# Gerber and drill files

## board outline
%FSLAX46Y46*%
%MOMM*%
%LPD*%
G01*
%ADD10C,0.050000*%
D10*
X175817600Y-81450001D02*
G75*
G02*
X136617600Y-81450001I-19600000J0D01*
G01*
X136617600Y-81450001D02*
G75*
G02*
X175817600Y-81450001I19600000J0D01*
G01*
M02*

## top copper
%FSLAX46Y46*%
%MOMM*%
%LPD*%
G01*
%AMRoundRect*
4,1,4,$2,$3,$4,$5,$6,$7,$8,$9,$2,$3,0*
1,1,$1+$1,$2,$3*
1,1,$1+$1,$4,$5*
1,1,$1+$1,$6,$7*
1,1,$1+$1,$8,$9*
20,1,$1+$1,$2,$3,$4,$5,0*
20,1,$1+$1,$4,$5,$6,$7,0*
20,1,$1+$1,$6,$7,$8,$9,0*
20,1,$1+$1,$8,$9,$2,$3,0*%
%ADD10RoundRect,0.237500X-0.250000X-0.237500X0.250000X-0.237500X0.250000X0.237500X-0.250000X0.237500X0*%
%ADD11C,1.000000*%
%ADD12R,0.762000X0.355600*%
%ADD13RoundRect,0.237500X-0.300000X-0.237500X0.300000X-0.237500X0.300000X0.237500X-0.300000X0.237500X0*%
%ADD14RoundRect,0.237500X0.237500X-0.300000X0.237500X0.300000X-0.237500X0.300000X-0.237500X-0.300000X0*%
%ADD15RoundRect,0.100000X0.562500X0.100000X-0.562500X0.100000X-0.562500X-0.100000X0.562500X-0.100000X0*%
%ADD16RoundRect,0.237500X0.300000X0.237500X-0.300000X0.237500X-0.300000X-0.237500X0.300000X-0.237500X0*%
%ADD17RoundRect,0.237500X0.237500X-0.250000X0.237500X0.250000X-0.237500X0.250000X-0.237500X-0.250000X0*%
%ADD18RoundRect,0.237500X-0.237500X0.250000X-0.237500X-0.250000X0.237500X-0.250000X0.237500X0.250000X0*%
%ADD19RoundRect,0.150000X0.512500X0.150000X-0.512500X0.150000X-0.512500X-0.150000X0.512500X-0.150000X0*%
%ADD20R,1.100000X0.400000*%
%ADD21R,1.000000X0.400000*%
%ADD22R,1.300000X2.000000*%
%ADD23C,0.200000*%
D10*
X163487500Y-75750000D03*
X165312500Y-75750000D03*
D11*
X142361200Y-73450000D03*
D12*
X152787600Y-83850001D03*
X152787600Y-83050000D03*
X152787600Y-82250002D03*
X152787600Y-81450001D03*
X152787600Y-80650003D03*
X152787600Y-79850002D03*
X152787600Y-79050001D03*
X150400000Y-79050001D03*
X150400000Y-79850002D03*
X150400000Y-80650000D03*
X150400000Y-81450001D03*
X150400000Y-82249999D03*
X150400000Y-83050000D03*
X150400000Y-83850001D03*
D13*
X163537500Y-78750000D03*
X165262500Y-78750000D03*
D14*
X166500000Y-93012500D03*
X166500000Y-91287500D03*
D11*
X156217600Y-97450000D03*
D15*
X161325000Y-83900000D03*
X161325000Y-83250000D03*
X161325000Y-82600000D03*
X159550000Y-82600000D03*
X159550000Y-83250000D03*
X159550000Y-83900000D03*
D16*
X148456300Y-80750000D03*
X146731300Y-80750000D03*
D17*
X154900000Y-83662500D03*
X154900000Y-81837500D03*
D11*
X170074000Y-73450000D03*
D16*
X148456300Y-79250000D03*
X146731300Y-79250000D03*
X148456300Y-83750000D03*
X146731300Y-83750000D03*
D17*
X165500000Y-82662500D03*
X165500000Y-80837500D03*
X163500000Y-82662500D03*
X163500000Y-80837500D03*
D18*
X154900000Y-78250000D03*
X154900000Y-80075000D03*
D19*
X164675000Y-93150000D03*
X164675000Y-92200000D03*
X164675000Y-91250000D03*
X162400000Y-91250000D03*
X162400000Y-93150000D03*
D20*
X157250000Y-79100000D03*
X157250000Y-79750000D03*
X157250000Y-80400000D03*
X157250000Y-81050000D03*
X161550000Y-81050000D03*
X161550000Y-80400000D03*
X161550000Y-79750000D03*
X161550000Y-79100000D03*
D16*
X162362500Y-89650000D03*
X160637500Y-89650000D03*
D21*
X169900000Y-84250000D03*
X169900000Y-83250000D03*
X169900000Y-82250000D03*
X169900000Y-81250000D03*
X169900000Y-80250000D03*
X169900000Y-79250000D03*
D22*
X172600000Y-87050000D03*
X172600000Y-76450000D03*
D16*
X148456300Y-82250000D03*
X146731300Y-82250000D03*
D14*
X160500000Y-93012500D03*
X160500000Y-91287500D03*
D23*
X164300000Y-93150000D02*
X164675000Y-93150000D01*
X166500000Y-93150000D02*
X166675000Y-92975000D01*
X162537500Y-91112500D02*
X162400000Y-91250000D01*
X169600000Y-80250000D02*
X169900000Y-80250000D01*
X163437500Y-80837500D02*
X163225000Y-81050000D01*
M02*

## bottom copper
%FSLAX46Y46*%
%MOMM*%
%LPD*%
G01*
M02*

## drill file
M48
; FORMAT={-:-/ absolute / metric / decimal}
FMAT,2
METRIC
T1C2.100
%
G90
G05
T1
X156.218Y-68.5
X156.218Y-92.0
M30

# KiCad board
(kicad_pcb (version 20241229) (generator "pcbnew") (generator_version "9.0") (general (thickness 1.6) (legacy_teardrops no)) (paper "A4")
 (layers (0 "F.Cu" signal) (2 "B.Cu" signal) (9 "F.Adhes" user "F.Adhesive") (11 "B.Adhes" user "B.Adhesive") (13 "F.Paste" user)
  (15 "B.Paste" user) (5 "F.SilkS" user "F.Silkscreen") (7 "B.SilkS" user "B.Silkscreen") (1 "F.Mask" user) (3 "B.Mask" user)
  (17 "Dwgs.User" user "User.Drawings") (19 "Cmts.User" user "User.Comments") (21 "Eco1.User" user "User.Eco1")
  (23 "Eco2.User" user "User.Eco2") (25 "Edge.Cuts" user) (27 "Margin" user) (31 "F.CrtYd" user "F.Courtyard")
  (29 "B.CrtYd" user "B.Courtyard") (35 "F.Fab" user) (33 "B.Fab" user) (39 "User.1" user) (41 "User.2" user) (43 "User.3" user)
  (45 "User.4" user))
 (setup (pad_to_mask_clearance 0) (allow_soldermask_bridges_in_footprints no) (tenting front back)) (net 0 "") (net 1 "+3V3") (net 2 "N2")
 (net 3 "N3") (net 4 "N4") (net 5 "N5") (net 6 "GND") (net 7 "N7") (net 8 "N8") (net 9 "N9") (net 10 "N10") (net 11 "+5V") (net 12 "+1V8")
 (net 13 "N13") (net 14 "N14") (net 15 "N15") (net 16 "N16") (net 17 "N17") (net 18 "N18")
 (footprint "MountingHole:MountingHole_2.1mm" (layer "F.Cu") (at 156.2176 68.5)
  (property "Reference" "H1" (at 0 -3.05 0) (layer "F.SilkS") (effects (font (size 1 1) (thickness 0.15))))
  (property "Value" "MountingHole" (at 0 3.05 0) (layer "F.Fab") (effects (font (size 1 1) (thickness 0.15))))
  (pad "" np_thru_hole circle (at 0 0) (size 2.1 2.1) (drill 2.1) (layers "*.Cu" "*.Mask")))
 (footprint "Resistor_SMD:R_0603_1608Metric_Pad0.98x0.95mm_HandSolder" (layer "F.Cu") (at 164.4 75.75)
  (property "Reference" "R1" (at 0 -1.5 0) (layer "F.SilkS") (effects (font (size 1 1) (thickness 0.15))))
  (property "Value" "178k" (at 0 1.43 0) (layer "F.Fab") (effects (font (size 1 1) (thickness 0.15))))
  (pad "1" smd roundrect (at -0.9125 0) (size 0.975 0.95) (layers "F.Cu" "F.Mask" "F.Paste") (roundrect_rratio 0.25) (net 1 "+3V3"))
  (pad "2" smd roundrect (at 0.9125 0) (size 0.975 0.95) (layers "F.Cu" "F.Mask" "F.Paste") (roundrect_rratio 0.25) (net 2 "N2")))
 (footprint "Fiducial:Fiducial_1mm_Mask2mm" (layer "F.Cu") (at 142.3612 73.45 180)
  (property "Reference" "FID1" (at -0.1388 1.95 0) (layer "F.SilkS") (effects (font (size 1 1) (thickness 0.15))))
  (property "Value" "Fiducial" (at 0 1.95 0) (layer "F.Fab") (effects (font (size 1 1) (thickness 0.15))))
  (pad "" smd circle (at 0 0 180) (size 1 1) (layers "F.Cu" "F.Mask") (solder_mask_margin 0.5) (clearance 0.6)))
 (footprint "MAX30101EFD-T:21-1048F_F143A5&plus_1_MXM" (layer "F.Cu") (at 151.5938 81.450001 180)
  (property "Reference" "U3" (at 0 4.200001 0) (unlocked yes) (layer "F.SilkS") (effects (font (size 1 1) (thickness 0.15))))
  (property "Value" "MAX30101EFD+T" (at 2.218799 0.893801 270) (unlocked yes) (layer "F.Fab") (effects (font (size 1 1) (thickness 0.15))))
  (pad "1" smd rect (at -1.1938 -2.4 180) (size 0.762 0.3556) (layers "F.Cu" "F.Mask" "F.Paste") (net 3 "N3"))
  (pad "2" smd rect (at -1.1938 -1.599999 180) (size 0.762 0.3556) (layers "F.Cu" "F.Mask" "F.Paste") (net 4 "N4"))
  (pad "3" smd rect (at -1.1938 -0.800001 180) (size 0.762 0.3556) (layers "F.Cu" "F.Mask" "F.Paste") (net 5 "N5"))
  (pad "4" smd rect (at -1.1938 0 180) (size 0.762 0.3556) (layers "F.Cu" "F.Mask" "F.Paste") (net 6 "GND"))
  (pad "5" smd rect (at -1.1938 0.799998 180) (size 0.762 0.3556) (layers "F.Cu" "F.Mask" "F.Paste") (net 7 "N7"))
  (pad "6" smd rect (at -1.1938 1.599999 180) (size 0.762 0.3556) (layers "F.Cu" "F.Mask" "F.Paste") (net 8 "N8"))
  (pad "7" smd rect (at -1.1938 2.4 180) (size 0.762 0.3556) (layers "F.Cu" "F.Mask" "F.Paste") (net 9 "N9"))
  (pad "8" smd rect (at 1.1938 2.4 180) (size 0.762 0.3556) (layers "F.Cu" "F.Mask" "F.Paste") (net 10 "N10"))
  (pad "9" smd rect (at 1.1938 1.599999 180) (size 0.762 0.3556) (layers "F.Cu" "F.Mask" "F.Paste") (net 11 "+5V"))
  (pad "10" smd rect (at 1.1938 0.800001 180) (size 0.762 0.3556) (layers "F.Cu" "F.Mask" "F.Paste") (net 11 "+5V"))
  (pad "11" smd rect (at 1.1938 0 180) (size 0.762 0.3556) (layers "F.Cu" "F.Mask" "F.Paste") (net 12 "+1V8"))
  (pad "12" smd rect (at 1.1938 -0.799998 180) (size 0.762 0.3556) (layers "F.Cu" "F.Mask" "F.Paste") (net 6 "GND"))
  (pad "13" smd rect (at 1.1938 -1.599999 180) (size 0.762 0.3556) (layers "F.Cu" "F.Mask" "F.Paste") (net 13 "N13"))
  (pad "14" smd rect (at 1.1938 -2.4 180) (size 0.762 0.3556) (layers "F.Cu" "F.Mask" "F.Paste") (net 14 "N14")))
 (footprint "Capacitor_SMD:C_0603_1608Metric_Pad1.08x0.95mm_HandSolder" (layer "F.Cu") (at 164.4 78.75)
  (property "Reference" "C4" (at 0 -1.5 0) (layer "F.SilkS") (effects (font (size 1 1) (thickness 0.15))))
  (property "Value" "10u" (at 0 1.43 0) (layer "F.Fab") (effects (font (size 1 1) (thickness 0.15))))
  (pad "1" smd roundrect (at -0.8625 0) (size 1.075 0.95) (layers "F.Cu" "F.Mask" "F.Paste") (roundrect_rratio 0.25) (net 2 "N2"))
  (pad "2" smd roundrect (at 0.8625 0) (size 1.075 0.95) (layers "F.Cu" "F.Mask" "F.Paste") (roundrect_rratio 0.25) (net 6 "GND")))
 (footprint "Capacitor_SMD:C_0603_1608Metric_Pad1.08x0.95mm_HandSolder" (layer "F.Cu") (at 166.5 92.15 90)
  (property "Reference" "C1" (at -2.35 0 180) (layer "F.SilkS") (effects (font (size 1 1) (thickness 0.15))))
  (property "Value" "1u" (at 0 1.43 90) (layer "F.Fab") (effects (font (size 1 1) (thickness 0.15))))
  (pad "1" smd roundrect (at -0.8625 0 90) (size 1.075 0.95) (layers "F.Cu" "F.Mask" "F.Paste") (roundrect_rratio 0.25) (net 1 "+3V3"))
  (pad "2" smd roundrect (at 0.8625 0 90) (size 1.075 0.95) (layers "F.Cu" "F.Mask" "F.Paste") (roundrect_rratio 0.25) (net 6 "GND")))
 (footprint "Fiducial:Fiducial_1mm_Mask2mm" (layer "F.Cu") (at 156.2176 97.45 180)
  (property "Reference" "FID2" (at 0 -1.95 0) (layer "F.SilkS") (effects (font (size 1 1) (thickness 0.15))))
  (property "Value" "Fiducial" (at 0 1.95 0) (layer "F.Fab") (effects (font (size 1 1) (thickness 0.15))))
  (pad "" smd circle (at 0 0 180) (size 1 1) (layers "F.Cu" "F.Mask") (solder_mask_margin 0.5) (clearance 0.6)))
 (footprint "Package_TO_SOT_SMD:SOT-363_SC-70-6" (layer "F.Cu") (at 160.4375 83.25 180)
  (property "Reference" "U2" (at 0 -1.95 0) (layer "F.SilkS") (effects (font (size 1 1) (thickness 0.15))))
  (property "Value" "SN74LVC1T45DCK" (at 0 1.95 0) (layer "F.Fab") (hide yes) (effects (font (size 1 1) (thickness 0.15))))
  (pad "1" smd roundrect (at -0.8875 -0.65 180) (size 1.325 0.4) (layers "F.Cu" "F.Mask" "F.Paste") (roundrect_rratio 0.25) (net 1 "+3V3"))
  (pad "2" smd roundrect (at -0.8875 0 180) (size 1.325 0.4) (layers "F.Cu" "F.Mask" "F.Paste") (roundrect_rratio 0.25) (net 6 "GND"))
  (pad "3" smd roundrect (at -0.8875 0.65 180) (size 1.325 0.4) (layers "F.Cu" "F.Mask" "F.Paste") (roundrect_rratio 0.25) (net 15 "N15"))
  (pad "4" smd roundrect (at 0.8875 0.65 180) (size 1.325 0.4) (layers "F.Cu" "F.Mask" "F.Paste") (roundrect_rratio 0.25) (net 13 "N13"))
  (pad "5" smd roundrect (at 0.8875 0 180) (size 1.325 0.4) (layers "F.Cu" "F.Mask" "F.Paste") (roundrect_rratio 0.25) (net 6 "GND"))
  (pad "6" smd roundrect (at 0.8875 -0.65 180) (size 1.325 0.4) (layers "F.Cu" "F.Mask" "F.Paste") (roundrect_rratio 0.25) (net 12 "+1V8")))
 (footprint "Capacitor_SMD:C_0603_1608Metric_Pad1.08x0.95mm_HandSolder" (layer "F.Cu") (at 147.5938 80.75 180)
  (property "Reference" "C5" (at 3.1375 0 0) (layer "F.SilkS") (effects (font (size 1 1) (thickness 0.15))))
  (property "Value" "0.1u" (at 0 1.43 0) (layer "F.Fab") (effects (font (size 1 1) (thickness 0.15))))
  (pad "1" smd roundrect (at -0.8625 0 180) (size 1.075 0.95) (layers "F.Cu" "F.Mask" "F.Paste") (roundrect_rratio 0.25) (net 11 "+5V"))
  (pad "2" smd roundrect (at 0.8625 0 180) (size 1.075 0.95) (layers "F.Cu" "F.Mask" "F.Paste") (roundrect_rratio 0.25) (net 6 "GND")))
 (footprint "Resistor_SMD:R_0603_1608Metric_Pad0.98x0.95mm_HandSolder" (layer "F.Cu") (at 154.9 82.75 90)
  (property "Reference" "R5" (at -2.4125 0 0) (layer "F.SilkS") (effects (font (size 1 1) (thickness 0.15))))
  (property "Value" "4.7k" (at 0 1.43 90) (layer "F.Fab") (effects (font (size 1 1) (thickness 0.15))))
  (pad "1" smd roundrect (at -0.9125 0 90) (size 0.975 0.95) (layers "F.Cu" "F.Mask" "F.Paste") (roundrect_rratio 0.25) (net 12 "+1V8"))
  (pad "2" smd roundrect (at 0.9125 0 90) (size 0.975 0.95) (layers "F.Cu" "F.Mask" "F.Paste") (roundrect_rratio 0.25) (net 5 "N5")))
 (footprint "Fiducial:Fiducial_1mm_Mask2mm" (layer "F.Cu") (at 170.074 73.45 180)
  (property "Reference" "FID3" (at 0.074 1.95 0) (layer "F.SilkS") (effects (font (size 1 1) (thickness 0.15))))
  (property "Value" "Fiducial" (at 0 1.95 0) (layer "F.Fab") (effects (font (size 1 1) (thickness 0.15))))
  (pad "" smd circle (at 0 0 180) (size 1 1) (layers "F.Cu" "F.Mask") (solder_mask_margin 0.5) (clearance 0.6)))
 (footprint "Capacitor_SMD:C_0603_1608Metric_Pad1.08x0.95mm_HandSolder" (layer "F.Cu") (at 147.5938 79.25 180)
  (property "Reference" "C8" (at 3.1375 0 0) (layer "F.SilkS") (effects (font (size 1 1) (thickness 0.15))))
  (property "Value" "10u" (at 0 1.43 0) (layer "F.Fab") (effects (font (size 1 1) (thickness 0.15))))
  (pad "1" smd roundrect (at -0.8625 0 180) (size 1.075 0.95) (layers "F.Cu" "F.Mask" "F.Paste") (roundrect_rratio 0.25) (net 11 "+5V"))
  (pad "2" smd roundrect (at 0.8625 0 180) (size 1.075 0.95) (layers "F.Cu" "F.Mask" "F.Paste") (roundrect_rratio 0.25) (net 6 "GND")))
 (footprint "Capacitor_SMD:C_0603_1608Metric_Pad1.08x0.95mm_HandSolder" (layer "F.Cu") (at 147.5938 83.75 180)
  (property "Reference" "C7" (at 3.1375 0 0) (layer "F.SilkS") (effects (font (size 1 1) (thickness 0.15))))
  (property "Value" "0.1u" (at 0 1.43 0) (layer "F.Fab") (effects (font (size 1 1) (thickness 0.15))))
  (pad "1" smd roundrect (at -0.8625 0 180) (size 1.075 0.95) (layers "F.Cu" "F.Mask" "F.Paste") (roundrect_rratio 0.25) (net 12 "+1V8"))
  (pad "2" smd roundrect (at 0.8625 0 180) (size 1.075 0.95) (layers "F.Cu" "F.Mask" "F.Paste") (roundrect_rratio 0.25) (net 6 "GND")))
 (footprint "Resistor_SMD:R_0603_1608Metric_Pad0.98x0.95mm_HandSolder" (layer "F.Cu") (at 165.5 81.75 90)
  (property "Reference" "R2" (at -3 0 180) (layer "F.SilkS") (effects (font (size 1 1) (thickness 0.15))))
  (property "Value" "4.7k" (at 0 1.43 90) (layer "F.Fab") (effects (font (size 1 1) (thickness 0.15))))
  (pad "1" smd roundrect (at -0.9125 0 90) (size 0.975 0.95) (layers "F.Cu" "F.Mask" "F.Paste") (roundrect_rratio 0.25) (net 1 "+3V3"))
  (pad "2" smd roundrect (at 0.9125 0 90) (size 0.975 0.95) (layers "F.Cu" "F.Mask" "F.Paste") (roundrect_rratio 0.25) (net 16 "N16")))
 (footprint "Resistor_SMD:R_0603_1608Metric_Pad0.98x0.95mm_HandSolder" (layer "F.Cu") (at 163.5 81.75 90)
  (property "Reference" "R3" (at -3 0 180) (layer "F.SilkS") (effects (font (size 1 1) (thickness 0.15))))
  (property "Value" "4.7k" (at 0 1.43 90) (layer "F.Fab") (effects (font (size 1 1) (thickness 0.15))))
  (pad "1" smd roundrect (at -0.9125 0 90) (size 0.975 0.95) (layers "F.Cu" "F.Mask" "F.Paste") (roundrect_rratio 0.25) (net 1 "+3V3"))
  (pad "2" smd roundrect (at 0.9125 0 90) (size 0.975 0.95) (layers "F.Cu" "F.Mask" "F.Paste") (roundrect_rratio 0.25) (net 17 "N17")))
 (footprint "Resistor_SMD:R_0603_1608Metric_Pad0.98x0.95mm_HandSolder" (layer "F.Cu") (at 154.9 79.1625 -90)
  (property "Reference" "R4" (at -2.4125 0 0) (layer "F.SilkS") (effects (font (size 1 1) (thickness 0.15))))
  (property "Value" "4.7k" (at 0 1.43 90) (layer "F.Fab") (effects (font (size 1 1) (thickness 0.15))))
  (pad "1" smd roundrect (at -0.9125 0 270) (size 0.975 0.95) (layers "F.Cu" "F.Mask" "F.Paste") (roundrect_rratio 0.25) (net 12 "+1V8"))
  (pad "2" smd roundrect (at 0.9125 0 270) (size 0.975 0.95) (layers "F.Cu" "F.Mask" "F.Paste") (roundrect_rratio 0.25) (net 4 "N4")))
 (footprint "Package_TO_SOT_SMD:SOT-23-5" (layer "F.Cu") (at 163.5375 92.2 180)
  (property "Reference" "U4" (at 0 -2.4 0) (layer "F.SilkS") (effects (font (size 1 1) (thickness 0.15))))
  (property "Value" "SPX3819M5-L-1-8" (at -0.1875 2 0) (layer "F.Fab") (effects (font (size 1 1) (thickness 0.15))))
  (pad "1" smd roundrect (at -1.1375 -0.95 180) (size 1.325 0.6) (layers "F.Cu" "F.Mask" "F.Paste") (roundrect_rratio 0.25) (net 1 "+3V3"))
  (pad "2" smd roundrect (at -1.1375 0 180) (size 1.325 0.6) (layers "F.Cu" "F.Mask" "F.Paste") (roundrect_rratio 0.25) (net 6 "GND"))
  (pad "3" smd roundrect (at -1.1375 0.95 180) (size 1.325 0.6) (layers "F.Cu" "F.Mask" "F.Paste") (roundrect_rratio 0.25) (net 1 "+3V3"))
  (pad "4" smd roundrect (at 1.1375 0.95 180) (size 1.325 0.6) (layers "F.Cu" "F.Mask" "F.Paste") (roundrect_rratio 0.25) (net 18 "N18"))
  (pad "5" smd roundrect (at 1.1375 -0.95 180) (size 1.325 0.6) (layers "F.Cu" "F.Mask" "F.Paste") (roundrect_rratio 0.25) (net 12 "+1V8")))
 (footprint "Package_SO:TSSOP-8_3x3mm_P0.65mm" (layer "F.Cu") (at 159.4 80.075)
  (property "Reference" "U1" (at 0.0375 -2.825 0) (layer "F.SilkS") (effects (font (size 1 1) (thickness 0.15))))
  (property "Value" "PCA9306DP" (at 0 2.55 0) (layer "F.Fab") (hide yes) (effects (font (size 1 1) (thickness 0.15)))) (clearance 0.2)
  (pad "1" smd rect (at -2.15 -0.975) (size 1.1 0.4) (layers "F.Cu" "F.Mask" "F.Paste") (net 6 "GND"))
  (pad "2" smd rect (at -2.15 -0.325) (size 1.1 0.4) (layers "F.Cu" "F.Mask" "F.Paste") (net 12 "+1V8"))
  (pad "3" smd rect (at -2.15 0.325) (size 1.1 0.4) (layers "F.Cu" "F.Mask" "F.Paste") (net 4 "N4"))
  (pad "4" smd rect (at -2.15 0.975) (size 1.1 0.4) (layers "F.Cu" "F.Mask" "F.Paste") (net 5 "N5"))
  (pad "5" smd rect (at 2.15 0.975) (size 1.1 0.4) (layers "F.Cu" "F.Mask" "F.Paste") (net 17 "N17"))
  (pad "6" smd rect (at 2.15 0.325) (size 1.1 0.4) (layers "F.Cu" "F.Mask" "F.Paste") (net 16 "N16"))
  (pad "7" smd rect (at 2.15 -0.325) (size 1.1 0.4) (layers "F.Cu" "F.Mask" "F.Paste") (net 1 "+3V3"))
  (pad "8" smd rect (at 2.15 -0.975) (size 1.1 0.4) (layers "F.Cu" "F.Mask" "F.Paste") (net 2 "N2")))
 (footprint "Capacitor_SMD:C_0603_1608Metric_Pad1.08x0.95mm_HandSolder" (layer "F.Cu") (at 161.5 89.65 180)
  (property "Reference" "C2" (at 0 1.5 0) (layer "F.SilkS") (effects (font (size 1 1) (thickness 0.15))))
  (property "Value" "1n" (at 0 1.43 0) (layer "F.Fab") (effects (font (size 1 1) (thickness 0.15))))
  (pad "1" smd roundrect (at -0.8625 0 180) (size 1.075 0.95) (layers "F.Cu" "F.Mask" "F.Paste") (roundrect_rratio 0.25) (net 18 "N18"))
  (pad "2" smd roundrect (at 0.8625 0 180) (size 1.075 0.95) (layers "F.Cu" "F.Mask" "F.Paste") (roundrect_rratio 0.25) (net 6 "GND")))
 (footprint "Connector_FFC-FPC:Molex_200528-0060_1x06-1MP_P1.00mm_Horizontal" (layer "F.Cu") (at 170.81 81.75 90)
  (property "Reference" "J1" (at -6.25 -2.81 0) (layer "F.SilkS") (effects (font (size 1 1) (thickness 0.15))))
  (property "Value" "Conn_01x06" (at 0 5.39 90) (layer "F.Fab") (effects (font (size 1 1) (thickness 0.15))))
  (pad "1" smd rect (at -2.5 -0.91 90) (size 0.4 1) (layers "F.Cu" "F.Mask" "F.Paste") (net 1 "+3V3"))
  (pad "2" smd rect (at -1.5 -0.91 90) (size 0.4 1) (layers "F.Cu" "F.Mask" "F.Paste") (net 11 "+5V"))
  (pad "3" smd rect (at -0.5 -0.91 90) (size 0.4 1) (layers "F.Cu" "F.Mask" "F.Paste") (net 15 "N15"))
  (pad "4" smd rect (at 0.5 -0.91 90) (size 0.4 1) (layers "F.Cu" "F.Mask" "F.Paste") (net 16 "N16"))
  (pad "5" smd rect (at 1.5 -0.91 90) (size 0.4 1) (layers "F.Cu" "F.Mask" "F.Paste") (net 17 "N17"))
  (pad "6" smd rect (at 2.5 -0.91 90) (size 0.4 1) (layers "F.Cu" "F.Mask" "F.Paste") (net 6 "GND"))
  (pad "MP" smd rect (at -5.3 1.79 90) (size 2 1.3) (layers "F.Cu" "F.Mask" "F.Paste"))
  (pad "MP" smd rect (at 5.3 1.79 90) (size 2 1.3) (layers "F.Cu" "F.Mask" "F.Paste")))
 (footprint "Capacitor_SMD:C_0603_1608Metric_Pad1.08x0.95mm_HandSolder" (layer "F.Cu") (at 147.5938 82.25 180)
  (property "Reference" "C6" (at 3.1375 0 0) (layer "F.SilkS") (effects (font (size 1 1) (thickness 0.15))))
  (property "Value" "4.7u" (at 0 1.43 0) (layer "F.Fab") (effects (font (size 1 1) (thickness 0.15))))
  (pad "1" smd roundrect (at -0.8625 0 180) (size 1.075 0.95) (layers "F.Cu" "F.Mask" "F.Paste") (roundrect_rratio 0.25) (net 12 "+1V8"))
  (pad "2" smd roundrect (at 0.8625 0 180) (size 1.075 0.95) (layers "F.Cu" "F.Mask" "F.Paste") (roundrect_rratio 0.25) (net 6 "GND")))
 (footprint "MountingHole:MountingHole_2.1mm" (layer "F.Cu") (at 156.2176 92)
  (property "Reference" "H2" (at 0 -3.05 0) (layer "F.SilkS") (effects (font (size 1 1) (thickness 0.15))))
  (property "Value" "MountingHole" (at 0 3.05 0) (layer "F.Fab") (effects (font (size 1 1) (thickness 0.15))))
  (pad "" np_thru_hole circle (at 0 0) (size 2.1 2.1) (drill 2.1) (layers "*.Cu" "*.Mask")))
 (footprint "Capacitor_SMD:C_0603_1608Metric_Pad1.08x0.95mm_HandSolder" (layer "F.Cu") (at 160.5 92.15 90)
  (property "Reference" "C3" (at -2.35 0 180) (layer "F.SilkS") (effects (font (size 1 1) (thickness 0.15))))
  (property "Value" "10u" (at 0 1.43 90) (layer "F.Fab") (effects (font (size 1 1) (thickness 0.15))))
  (pad "1" smd roundrect (at -0.8625 0 90) (size 1.075 0.95) (layers "F.Cu" "F.Mask" "F.Paste") (roundrect_rratio 0.25) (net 12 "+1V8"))
  (pad "2" smd roundrect (at 0.8625 0 90) (size 1.075 0.95) (layers "F.Cu" "F.Mask" "F.Paste") (roundrect_rratio 0.25) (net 6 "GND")))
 (gr_circle (center 156.2176 81.450001) (end 136.6176 81.450001) (stroke (width 0.05) (type solid)) (fill no) (layer "Edge.Cuts"))
 (segment (start 164.3 93.15) (end 164.675 93.15) (width 0.2) (layer "F.Cu") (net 1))
 (segment (start 166.5 93.15) (end 166.675 92.975) (width 0.2) (layer "F.Cu") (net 1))
 (segment (start 162.5375 91.1125) (end 162.4 91.25) (width 0.2) (layer "F.Cu") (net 18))
 (segment (start 169.6 80.25) (end 169.9 80.25) (width 0.2) (layer "F.Cu") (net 17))
 (segment (start 163.4375 80.8375) (end 163.225 81.05) (width 0.2) (layer "F.Cu") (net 17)))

